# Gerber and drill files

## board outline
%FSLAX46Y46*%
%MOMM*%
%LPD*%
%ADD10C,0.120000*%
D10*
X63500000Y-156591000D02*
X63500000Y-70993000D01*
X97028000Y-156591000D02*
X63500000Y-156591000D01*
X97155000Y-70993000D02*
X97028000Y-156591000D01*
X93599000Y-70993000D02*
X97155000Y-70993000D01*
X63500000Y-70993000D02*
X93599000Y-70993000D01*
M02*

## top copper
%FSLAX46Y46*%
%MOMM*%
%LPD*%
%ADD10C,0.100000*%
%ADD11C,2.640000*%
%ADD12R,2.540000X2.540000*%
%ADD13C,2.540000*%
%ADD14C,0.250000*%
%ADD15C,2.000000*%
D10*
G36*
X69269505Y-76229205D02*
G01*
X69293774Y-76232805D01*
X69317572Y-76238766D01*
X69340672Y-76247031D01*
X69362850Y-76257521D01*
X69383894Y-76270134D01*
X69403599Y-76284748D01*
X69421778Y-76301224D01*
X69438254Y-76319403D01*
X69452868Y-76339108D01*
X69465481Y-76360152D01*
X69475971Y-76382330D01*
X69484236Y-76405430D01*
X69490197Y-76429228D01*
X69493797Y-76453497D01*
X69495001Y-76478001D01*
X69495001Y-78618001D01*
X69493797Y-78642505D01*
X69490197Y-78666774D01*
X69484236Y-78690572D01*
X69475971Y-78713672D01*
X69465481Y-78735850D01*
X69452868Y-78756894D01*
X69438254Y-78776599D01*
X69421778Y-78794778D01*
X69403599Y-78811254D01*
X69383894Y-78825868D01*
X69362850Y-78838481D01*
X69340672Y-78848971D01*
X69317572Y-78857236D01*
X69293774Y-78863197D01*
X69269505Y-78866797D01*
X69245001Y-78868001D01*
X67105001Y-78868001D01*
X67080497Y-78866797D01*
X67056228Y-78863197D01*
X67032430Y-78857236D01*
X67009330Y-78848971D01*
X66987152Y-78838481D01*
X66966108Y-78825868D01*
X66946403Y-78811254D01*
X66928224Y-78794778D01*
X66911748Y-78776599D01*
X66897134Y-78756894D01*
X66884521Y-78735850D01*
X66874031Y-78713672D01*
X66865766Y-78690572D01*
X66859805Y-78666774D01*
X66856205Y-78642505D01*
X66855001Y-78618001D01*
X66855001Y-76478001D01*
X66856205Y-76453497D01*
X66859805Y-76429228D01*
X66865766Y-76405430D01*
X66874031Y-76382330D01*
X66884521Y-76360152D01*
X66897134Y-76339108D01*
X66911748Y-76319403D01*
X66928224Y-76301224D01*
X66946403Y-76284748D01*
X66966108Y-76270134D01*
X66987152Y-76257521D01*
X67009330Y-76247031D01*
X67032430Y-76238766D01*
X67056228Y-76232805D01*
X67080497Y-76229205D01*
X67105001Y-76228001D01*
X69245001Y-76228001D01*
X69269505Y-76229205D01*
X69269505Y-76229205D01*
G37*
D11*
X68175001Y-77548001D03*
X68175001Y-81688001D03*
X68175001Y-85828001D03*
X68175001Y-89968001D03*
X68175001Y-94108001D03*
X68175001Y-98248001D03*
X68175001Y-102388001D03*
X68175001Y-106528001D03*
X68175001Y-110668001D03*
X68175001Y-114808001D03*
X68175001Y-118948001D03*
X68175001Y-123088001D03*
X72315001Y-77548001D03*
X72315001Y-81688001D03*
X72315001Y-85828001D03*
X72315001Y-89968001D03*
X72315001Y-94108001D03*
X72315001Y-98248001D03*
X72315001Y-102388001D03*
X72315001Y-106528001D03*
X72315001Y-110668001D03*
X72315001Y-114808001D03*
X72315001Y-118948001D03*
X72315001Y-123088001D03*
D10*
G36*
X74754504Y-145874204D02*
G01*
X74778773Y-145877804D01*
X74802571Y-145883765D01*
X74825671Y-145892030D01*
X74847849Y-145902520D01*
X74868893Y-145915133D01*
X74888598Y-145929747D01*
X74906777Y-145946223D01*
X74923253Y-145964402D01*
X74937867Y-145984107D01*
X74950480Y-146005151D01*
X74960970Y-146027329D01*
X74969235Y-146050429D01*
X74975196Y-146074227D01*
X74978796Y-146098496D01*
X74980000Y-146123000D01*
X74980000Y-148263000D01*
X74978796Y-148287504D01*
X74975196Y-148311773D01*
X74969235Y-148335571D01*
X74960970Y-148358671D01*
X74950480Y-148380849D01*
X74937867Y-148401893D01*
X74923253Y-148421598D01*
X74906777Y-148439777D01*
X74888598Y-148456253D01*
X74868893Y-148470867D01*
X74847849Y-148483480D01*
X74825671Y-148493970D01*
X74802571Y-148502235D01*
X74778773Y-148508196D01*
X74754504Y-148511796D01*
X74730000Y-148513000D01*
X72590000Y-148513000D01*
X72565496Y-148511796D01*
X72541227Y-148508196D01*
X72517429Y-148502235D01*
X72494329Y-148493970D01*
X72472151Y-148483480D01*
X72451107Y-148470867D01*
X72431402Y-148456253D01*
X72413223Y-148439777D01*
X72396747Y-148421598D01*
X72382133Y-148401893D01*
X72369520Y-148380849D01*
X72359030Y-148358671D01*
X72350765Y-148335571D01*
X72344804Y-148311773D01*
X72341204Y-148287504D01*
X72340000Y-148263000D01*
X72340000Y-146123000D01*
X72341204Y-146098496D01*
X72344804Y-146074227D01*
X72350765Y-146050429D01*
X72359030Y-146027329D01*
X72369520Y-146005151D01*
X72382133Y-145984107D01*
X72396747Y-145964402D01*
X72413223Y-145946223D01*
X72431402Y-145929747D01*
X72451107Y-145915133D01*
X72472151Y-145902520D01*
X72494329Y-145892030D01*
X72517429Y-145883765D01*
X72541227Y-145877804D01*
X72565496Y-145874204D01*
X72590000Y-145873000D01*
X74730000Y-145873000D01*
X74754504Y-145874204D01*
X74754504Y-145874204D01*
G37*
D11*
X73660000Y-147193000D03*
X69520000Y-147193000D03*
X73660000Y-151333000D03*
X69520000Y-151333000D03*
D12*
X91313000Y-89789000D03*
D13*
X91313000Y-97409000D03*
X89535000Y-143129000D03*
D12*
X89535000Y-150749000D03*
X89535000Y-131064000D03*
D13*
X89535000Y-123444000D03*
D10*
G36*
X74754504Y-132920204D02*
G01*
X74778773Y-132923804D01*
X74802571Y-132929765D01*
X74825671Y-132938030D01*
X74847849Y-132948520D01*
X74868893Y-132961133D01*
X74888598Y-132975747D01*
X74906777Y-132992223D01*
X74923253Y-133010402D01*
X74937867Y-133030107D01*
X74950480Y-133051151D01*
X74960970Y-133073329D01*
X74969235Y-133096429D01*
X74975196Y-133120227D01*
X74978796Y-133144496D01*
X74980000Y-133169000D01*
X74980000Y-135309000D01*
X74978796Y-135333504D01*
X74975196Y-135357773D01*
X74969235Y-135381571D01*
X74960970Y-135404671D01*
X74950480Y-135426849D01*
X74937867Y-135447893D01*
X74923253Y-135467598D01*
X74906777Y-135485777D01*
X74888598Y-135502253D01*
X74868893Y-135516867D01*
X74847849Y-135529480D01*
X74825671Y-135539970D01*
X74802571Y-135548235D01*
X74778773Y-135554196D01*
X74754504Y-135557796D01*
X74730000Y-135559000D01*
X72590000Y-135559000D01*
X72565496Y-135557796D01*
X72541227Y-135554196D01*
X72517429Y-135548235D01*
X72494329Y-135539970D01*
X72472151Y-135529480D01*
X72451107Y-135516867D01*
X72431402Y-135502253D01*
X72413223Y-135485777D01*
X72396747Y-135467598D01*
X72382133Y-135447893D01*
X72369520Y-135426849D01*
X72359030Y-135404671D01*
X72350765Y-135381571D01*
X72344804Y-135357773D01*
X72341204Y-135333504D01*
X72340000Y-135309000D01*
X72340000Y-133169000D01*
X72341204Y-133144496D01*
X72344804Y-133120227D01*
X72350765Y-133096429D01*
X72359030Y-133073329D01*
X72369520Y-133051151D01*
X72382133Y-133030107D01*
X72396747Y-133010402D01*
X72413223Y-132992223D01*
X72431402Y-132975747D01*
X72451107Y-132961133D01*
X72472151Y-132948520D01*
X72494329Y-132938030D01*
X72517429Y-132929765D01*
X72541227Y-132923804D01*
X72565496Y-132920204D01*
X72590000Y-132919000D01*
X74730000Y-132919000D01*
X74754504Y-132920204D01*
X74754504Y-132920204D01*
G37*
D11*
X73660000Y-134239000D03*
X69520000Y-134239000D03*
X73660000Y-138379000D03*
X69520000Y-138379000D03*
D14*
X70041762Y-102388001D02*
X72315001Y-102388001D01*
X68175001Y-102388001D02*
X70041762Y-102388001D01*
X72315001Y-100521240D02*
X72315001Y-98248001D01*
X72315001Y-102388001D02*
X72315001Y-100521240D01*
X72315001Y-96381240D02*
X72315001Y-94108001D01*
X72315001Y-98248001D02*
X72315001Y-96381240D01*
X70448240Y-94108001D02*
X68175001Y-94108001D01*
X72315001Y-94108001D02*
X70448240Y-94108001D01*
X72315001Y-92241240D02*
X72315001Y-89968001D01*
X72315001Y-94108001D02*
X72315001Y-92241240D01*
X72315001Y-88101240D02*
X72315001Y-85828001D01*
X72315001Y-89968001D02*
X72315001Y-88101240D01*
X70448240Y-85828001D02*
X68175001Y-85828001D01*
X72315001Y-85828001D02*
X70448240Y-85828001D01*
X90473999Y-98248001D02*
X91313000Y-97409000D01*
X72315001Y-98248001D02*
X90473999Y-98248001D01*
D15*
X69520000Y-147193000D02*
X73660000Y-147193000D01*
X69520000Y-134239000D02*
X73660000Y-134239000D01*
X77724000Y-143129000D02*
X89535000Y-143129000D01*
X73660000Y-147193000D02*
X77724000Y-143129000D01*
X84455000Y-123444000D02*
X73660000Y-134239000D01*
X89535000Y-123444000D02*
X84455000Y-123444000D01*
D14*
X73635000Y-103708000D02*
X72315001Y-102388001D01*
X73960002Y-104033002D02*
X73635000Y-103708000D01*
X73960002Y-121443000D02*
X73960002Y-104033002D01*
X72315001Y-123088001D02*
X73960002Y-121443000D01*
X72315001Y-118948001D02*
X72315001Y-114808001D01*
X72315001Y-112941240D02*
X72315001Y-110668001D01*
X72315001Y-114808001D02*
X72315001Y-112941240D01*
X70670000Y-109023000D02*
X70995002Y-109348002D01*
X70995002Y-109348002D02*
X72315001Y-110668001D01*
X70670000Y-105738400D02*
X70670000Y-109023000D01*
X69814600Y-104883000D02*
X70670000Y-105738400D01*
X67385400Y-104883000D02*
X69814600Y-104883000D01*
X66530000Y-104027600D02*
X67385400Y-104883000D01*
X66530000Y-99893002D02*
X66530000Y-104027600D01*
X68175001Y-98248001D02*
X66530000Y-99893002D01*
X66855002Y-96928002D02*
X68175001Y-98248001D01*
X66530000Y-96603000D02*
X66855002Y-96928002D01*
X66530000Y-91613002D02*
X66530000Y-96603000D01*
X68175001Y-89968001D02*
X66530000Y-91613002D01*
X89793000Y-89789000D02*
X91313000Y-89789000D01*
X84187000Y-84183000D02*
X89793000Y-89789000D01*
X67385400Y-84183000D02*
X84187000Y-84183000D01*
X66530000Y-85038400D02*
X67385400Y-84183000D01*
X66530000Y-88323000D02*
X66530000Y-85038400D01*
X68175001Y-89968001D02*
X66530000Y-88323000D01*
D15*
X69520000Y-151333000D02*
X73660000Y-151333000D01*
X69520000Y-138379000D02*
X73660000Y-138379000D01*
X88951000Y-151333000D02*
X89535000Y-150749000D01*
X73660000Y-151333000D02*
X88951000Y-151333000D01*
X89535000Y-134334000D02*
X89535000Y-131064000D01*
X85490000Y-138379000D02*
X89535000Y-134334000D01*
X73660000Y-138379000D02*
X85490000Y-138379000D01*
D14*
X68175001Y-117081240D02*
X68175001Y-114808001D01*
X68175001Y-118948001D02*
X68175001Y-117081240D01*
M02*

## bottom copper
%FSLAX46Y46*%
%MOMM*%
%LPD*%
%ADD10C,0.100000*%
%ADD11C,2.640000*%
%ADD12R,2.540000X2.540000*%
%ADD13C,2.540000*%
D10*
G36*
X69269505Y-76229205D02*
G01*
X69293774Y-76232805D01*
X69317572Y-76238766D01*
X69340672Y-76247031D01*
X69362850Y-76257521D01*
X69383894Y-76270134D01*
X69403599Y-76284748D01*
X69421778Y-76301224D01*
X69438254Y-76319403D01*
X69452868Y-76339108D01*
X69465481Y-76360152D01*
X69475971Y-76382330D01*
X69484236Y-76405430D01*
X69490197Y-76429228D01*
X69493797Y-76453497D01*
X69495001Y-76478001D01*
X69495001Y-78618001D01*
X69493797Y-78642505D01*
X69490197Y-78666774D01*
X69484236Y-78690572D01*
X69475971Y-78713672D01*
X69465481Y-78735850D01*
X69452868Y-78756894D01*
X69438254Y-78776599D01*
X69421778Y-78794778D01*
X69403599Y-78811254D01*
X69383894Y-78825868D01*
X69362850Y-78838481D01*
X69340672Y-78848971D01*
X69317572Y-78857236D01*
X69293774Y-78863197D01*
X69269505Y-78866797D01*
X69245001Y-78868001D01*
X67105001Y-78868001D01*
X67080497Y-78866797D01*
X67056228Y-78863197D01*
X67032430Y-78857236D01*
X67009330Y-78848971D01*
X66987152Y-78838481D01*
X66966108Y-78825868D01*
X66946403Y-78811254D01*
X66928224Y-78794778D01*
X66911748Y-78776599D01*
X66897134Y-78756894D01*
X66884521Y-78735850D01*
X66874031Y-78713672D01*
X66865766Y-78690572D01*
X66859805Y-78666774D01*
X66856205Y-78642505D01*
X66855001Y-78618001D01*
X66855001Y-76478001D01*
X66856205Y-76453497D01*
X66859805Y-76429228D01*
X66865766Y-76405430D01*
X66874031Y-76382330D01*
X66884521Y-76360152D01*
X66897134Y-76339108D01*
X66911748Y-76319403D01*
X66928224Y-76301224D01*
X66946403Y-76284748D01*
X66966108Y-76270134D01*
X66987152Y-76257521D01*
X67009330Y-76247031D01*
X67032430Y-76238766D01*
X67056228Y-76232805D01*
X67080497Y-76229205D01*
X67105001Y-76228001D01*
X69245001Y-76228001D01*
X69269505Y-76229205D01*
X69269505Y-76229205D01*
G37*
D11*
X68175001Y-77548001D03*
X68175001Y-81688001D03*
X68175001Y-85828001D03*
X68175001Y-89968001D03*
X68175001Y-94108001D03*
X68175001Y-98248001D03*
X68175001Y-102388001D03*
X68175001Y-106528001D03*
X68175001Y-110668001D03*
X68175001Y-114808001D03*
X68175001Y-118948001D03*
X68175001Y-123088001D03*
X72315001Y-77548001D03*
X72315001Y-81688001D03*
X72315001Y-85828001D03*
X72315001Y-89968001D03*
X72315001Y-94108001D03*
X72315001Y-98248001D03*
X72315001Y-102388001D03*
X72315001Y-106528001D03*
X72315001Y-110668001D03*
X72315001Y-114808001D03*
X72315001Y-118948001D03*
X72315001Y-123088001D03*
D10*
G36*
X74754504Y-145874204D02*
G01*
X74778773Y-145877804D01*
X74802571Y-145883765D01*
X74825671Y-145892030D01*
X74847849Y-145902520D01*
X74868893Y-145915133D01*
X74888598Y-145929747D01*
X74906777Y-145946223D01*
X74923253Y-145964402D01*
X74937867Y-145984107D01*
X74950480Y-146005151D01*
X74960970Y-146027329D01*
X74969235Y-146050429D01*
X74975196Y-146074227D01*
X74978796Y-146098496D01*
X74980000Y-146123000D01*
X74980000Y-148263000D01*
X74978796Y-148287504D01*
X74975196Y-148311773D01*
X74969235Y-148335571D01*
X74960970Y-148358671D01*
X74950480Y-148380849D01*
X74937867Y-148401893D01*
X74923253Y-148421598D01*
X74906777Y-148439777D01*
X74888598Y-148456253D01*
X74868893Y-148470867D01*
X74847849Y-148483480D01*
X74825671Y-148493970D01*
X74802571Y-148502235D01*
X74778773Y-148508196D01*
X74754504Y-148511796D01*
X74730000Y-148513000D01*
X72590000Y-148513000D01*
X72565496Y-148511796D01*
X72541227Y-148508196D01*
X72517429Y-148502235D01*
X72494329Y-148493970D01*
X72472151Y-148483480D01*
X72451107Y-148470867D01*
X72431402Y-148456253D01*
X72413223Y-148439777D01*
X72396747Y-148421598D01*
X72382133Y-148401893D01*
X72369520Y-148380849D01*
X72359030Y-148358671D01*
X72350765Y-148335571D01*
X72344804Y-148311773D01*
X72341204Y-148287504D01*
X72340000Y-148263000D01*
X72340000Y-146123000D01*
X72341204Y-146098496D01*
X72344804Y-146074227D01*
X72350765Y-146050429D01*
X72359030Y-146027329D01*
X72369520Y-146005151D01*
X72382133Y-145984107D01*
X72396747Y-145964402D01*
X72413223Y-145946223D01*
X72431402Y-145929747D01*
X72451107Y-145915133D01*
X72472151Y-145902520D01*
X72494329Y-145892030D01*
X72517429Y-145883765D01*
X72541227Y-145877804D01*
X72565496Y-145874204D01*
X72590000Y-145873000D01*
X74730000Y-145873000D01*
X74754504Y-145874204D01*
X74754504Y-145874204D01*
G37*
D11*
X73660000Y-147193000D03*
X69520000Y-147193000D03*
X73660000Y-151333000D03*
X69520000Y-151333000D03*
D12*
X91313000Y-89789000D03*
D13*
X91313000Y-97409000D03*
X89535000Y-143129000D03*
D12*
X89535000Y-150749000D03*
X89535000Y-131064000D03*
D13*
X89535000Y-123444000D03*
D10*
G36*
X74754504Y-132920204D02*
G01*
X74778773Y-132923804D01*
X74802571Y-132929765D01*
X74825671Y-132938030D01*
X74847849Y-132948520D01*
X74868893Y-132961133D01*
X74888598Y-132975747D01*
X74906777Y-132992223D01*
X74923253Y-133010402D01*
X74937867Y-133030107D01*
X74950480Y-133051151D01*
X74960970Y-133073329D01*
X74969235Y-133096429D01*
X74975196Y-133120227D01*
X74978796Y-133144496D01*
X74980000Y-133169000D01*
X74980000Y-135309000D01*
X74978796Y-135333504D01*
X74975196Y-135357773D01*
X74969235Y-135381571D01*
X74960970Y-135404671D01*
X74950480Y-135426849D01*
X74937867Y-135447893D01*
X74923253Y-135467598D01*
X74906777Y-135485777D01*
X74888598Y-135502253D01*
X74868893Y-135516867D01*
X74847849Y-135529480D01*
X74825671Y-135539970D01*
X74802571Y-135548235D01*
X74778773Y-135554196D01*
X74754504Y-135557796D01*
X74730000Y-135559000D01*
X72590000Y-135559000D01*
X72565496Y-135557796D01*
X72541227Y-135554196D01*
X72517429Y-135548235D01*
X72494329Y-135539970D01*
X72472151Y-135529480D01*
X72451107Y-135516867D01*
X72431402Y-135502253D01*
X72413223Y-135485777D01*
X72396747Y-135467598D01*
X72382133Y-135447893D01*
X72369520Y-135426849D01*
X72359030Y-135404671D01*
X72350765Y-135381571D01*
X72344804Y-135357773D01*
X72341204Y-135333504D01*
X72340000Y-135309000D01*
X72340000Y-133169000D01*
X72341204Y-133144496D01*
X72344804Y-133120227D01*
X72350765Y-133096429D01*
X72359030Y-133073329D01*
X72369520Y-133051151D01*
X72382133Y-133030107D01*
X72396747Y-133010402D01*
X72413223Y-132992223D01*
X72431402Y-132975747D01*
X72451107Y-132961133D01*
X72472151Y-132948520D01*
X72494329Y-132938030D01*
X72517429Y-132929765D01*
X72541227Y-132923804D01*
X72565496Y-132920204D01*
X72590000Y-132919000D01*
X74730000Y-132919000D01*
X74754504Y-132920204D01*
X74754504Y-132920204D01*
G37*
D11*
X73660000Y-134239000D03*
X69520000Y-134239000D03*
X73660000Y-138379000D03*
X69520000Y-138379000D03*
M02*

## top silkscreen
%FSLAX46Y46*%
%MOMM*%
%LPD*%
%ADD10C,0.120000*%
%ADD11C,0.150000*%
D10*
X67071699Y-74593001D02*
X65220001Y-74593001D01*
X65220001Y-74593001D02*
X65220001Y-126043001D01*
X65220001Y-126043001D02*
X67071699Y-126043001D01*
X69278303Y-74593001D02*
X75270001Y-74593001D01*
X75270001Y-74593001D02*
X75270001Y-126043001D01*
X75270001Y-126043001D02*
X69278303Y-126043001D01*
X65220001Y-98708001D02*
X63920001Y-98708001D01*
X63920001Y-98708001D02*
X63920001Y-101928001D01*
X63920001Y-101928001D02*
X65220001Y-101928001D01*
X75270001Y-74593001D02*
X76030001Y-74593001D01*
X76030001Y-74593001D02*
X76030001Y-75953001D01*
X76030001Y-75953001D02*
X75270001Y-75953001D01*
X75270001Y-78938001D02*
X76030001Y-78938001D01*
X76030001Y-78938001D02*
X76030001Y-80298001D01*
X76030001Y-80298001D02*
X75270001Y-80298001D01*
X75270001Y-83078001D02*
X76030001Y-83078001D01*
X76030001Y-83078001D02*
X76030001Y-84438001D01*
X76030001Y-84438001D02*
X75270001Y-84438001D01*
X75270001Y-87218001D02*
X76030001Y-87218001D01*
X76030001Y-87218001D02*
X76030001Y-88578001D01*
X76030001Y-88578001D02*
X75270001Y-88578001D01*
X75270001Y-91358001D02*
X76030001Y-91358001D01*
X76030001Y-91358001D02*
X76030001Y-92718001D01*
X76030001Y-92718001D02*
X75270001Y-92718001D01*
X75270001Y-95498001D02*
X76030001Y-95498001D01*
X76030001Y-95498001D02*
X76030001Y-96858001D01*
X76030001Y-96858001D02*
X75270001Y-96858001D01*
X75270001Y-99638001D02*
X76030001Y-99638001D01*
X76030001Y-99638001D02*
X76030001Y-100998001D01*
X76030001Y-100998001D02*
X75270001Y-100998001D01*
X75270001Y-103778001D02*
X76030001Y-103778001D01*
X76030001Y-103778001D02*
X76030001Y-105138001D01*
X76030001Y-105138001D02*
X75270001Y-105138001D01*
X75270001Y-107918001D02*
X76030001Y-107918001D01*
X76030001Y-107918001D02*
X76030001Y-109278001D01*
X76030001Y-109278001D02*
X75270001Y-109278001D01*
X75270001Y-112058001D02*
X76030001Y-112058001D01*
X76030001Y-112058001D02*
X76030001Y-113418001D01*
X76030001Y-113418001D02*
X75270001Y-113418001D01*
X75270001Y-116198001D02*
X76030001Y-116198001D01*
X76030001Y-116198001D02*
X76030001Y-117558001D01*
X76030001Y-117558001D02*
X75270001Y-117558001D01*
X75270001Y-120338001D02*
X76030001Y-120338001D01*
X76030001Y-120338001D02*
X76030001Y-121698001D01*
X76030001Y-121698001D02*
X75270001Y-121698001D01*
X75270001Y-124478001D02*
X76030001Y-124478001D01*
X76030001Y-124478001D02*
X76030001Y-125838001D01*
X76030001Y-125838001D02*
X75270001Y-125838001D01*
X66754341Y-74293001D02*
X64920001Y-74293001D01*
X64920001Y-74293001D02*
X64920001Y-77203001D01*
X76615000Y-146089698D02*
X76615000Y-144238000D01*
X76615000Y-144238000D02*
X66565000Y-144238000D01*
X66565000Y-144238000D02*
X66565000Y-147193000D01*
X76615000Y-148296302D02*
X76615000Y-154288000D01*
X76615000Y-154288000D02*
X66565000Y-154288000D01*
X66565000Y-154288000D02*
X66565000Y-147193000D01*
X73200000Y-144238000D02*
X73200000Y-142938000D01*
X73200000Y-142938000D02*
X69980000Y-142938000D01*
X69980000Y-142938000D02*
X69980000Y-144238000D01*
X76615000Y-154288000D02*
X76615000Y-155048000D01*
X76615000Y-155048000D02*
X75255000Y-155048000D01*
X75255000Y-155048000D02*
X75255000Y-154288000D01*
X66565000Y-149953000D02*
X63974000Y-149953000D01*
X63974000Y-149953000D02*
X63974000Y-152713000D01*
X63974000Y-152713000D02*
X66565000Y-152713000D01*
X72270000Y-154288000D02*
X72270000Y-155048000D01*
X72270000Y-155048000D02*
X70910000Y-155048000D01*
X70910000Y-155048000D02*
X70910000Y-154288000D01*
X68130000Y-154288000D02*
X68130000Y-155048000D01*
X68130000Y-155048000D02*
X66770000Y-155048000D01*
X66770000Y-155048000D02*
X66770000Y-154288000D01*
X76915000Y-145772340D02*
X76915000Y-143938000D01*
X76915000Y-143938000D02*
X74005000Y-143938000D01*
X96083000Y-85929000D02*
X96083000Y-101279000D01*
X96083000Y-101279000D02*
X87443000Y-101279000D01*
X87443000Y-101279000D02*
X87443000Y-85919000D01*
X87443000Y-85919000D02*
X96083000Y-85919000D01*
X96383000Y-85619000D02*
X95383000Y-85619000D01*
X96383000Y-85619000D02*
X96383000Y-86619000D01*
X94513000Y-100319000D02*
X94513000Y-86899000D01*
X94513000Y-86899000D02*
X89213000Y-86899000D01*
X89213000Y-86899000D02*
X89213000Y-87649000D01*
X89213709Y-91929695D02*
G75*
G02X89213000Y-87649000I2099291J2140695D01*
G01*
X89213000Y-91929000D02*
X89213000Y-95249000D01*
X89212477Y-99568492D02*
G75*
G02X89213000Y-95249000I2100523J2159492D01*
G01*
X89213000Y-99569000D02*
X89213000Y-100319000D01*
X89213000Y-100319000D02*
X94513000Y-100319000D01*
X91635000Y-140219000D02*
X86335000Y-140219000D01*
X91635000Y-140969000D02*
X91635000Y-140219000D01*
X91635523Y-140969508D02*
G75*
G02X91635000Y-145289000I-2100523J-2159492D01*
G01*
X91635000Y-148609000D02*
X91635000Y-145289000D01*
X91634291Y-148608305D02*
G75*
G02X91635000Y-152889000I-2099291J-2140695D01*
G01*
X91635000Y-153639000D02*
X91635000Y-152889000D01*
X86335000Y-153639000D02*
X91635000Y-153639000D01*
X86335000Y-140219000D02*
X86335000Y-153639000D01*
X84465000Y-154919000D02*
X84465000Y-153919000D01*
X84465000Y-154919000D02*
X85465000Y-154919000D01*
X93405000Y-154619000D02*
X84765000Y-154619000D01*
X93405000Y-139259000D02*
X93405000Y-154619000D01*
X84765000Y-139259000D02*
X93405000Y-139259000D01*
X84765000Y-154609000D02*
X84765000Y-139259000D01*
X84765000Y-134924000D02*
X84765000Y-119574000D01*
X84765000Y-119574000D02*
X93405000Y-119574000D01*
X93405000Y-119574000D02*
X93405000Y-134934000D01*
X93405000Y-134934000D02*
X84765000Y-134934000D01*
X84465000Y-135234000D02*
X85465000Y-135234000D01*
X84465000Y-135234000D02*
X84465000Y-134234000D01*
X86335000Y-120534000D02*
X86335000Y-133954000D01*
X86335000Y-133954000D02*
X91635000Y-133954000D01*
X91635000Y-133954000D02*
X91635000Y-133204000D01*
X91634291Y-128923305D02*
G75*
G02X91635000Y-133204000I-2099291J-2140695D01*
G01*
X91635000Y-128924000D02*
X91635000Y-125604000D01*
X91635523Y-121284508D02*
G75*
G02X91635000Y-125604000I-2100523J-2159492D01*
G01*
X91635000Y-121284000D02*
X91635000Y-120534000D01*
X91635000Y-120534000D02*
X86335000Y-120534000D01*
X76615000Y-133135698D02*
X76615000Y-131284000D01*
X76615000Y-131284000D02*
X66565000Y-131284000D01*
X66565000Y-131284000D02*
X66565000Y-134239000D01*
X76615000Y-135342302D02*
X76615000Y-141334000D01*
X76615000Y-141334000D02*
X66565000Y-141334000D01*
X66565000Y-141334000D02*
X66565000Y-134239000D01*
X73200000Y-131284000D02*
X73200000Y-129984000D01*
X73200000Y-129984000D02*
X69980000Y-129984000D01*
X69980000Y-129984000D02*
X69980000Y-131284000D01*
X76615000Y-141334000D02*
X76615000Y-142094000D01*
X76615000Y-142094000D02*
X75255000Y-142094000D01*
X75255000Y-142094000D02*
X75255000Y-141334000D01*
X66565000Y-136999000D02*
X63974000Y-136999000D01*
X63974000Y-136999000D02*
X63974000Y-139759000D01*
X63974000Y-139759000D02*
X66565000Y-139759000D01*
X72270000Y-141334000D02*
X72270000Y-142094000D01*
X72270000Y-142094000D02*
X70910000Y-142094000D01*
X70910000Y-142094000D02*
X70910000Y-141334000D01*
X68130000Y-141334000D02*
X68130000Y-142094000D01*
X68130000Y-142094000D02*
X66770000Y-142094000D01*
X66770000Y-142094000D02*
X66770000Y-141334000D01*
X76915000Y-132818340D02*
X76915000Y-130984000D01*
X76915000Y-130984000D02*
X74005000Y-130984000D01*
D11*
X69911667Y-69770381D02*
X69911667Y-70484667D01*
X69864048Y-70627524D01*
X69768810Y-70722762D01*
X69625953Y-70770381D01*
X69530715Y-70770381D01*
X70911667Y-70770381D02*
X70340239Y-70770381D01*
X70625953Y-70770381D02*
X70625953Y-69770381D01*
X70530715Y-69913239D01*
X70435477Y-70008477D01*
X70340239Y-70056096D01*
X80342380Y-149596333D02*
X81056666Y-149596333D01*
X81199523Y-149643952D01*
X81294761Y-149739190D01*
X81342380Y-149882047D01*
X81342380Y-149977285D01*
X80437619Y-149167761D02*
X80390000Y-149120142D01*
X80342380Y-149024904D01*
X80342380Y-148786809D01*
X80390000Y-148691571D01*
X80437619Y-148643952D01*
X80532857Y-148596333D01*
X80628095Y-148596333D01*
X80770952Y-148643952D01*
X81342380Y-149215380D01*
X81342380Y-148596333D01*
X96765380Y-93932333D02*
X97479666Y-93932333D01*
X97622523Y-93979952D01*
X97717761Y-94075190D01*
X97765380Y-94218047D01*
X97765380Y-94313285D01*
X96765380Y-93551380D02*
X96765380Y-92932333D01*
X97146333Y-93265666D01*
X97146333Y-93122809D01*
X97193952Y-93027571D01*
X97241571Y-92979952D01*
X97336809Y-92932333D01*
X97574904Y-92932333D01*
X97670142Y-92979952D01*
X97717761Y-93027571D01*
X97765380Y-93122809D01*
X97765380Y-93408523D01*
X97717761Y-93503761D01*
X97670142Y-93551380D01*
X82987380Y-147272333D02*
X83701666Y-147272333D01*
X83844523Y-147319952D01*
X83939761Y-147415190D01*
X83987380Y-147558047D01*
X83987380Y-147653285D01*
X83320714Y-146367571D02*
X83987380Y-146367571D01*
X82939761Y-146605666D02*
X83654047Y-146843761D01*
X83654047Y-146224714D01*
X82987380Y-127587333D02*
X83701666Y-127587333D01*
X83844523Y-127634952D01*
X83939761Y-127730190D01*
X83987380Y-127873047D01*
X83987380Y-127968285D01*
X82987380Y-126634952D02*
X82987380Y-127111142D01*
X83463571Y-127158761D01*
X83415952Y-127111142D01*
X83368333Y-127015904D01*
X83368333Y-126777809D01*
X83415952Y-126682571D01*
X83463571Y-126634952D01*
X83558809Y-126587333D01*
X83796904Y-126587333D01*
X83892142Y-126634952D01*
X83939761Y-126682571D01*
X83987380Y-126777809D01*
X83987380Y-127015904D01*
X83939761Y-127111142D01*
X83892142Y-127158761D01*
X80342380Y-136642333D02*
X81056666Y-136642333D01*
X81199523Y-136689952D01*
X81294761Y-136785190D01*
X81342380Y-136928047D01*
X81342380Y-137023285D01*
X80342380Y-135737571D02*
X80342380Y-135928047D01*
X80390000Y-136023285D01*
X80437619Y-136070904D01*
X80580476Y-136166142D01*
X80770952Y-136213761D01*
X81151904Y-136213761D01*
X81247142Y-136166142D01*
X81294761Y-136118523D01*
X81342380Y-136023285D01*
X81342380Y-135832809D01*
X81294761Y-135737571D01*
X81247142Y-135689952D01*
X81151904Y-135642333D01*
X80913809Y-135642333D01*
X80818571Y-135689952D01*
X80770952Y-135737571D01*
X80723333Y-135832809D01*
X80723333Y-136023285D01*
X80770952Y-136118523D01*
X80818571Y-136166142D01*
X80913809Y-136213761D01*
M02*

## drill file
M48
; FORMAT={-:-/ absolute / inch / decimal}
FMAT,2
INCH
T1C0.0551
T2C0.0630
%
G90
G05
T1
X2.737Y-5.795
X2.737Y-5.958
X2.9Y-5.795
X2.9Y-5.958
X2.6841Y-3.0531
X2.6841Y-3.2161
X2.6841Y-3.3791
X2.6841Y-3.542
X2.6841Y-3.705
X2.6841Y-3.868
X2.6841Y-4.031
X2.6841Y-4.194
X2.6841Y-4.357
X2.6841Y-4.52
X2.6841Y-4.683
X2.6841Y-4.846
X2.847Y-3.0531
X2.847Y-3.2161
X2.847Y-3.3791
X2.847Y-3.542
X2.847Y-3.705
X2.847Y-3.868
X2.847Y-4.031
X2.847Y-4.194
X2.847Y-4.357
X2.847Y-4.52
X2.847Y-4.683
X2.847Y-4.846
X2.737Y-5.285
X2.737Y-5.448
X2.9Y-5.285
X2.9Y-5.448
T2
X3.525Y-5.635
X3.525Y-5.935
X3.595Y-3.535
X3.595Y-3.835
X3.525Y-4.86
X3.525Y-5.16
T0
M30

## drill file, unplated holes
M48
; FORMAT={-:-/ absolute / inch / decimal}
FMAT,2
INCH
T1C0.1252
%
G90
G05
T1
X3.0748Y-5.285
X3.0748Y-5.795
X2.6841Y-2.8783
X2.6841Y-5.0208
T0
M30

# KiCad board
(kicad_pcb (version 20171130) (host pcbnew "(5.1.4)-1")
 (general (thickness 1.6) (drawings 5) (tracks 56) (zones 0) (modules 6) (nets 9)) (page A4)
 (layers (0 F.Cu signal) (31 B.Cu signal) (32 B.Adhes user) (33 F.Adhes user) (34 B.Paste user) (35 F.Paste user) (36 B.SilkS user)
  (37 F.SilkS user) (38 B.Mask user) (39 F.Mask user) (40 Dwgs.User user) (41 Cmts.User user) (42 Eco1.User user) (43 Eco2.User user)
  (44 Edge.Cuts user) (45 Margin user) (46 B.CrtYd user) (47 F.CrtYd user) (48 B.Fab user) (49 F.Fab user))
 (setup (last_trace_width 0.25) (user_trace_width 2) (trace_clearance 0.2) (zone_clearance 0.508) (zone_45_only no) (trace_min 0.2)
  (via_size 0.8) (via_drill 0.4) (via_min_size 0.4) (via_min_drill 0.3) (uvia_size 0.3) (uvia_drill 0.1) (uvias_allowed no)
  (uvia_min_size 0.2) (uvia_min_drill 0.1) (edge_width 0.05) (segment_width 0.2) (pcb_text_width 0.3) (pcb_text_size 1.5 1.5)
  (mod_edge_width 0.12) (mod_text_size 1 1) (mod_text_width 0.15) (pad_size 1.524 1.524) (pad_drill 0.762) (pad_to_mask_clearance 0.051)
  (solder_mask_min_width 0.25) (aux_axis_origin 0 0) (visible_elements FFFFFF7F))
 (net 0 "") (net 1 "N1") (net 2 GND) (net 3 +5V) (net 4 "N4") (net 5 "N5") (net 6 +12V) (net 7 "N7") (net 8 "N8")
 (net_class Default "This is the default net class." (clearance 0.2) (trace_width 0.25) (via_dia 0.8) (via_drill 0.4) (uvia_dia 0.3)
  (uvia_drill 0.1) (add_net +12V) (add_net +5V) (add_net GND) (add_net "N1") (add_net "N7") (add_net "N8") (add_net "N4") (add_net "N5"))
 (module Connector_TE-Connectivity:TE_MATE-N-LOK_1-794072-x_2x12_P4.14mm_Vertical (layer F.Cu) (at 68.175001 77.548001)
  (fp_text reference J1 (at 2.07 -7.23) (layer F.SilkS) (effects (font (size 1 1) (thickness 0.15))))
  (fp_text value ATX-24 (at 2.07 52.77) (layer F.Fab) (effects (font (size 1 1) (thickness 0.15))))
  (fp_line (start -1.103302 -2.955) (end -2.955 -2.955) (layer F.SilkS) (width 0.12))
  (fp_line (start -2.955 -2.955) (end -2.955 48.495) (layer F.SilkS) (width 0.12))
  (fp_line (start -2.955 48.495) (end -1.103302 48.495) (layer F.SilkS) (width 0.12))
  (fp_line (start 1.103302 -2.955) (end 7.095 -2.955) (layer F.SilkS) (width 0.12))
  (fp_line (start 7.095 -2.955) (end 7.095 48.495) (layer F.SilkS) (width 0.12))
  (fp_line (start 7.095 48.495) (end 1.103302 48.495) (layer F.SilkS) (width 0.12))
  (fp_line (start -2.955 21.16) (end -4.255 21.16) (layer F.SilkS) (width 0.12))
  (fp_line (start -4.255 21.16) (end -4.255 24.38) (layer F.SilkS) (width 0.12))
  (fp_line (start -4.255 24.38) (end -2.955 24.38) (layer F.SilkS) (width 0.12))
  (fp_line (start 7.095 -2.955) (end 7.855 -2.955) (layer F.SilkS) (width 0.12))
  (fp_line (start 7.855 -2.955) (end 7.855 -1.595) (layer F.SilkS) (width 0.12))
  (fp_line (start 7.855 -1.595) (end 7.095 -1.595) (layer F.SilkS) (width 0.12))
  (fp_line (start 7.095 1.39) (end 7.855 1.39) (layer F.SilkS) (width 0.12))
  (fp_line (start 7.855 1.39) (end 7.855 2.75) (layer F.SilkS) (width 0.12))
  (fp_line (start 7.855 2.75) (end 7.095 2.75) (layer F.SilkS) (width 0.12))
  (fp_line (start 7.095 5.53) (end 7.855 5.53) (layer F.SilkS) (width 0.12))
  (fp_line (start 7.855 5.53) (end 7.855 6.89) (layer F.SilkS) (width 0.12))
  (fp_line (start 7.855 6.89) (end 7.095 6.89) (layer F.SilkS) (width 0.12))
  (fp_line (start 7.095 9.67) (end 7.855 9.67) (layer F.SilkS) (width 0.12))
  (fp_line (start 7.855 9.67) (end 7.855 11.03) (layer F.SilkS) (width 0.12))
  (fp_line (start 7.855 11.03) (end 7.095 11.03) (layer F.SilkS) (width 0.12))
  (fp_line (start 7.095 13.81) (end 7.855 13.81) (layer F.SilkS) (width 0.12))
  (fp_line (start 7.855 13.81) (end 7.855 15.17) (layer F.SilkS) (width 0.12))
  (fp_line (start 7.855 15.17) (end 7.095 15.17) (layer F.SilkS) (width 0.12))
  (fp_line (start 7.095 17.95) (end 7.855 17.95) (layer F.SilkS) (width 0.12))
  (fp_line (start 7.855 17.95) (end 7.855 19.31) (layer F.SilkS) (width 0.12))
  (fp_line (start 7.855 19.31) (end 7.095 19.31) (layer F.SilkS) (width 0.12))
  (fp_line (start 7.095 22.09) (end 7.855 22.09) (layer F.SilkS) (width 0.12))
  (fp_line (start 7.855 22.09) (end 7.855 23.45) (layer F.SilkS) (width 0.12))
  (fp_line (start 7.855 23.45) (end 7.095 23.45) (layer F.SilkS) (width 0.12))
  (fp_line (start 7.095 26.23) (end 7.855 26.23) (layer F.SilkS) (width 0.12))
  (fp_line (start 7.855 26.23) (end 7.855 27.59) (layer F.SilkS) (width 0.12))
  (fp_line (start 7.855 27.59) (end 7.095 27.59) (layer F.SilkS) (width 0.12))
  (fp_line (start 7.095 30.37) (end 7.855 30.37) (layer F.SilkS) (width 0.12))
  (fp_line (start 7.855 30.37) (end 7.855 31.73) (layer F.SilkS) (width 0.12))
  (fp_line (start 7.855 31.73) (end 7.095 31.73) (layer F.SilkS) (width 0.12))
  (fp_line (start 7.095 34.51) (end 7.855 34.51) (layer F.SilkS) (width 0.12))
  (fp_line (start 7.855 34.51) (end 7.855 35.87) (layer F.SilkS) (width 0.12))
  (fp_line (start 7.855 35.87) (end 7.095 35.87) (layer F.SilkS) (width 0.12))
  (fp_line (start 7.095 38.65) (end 7.855 38.65) (layer F.SilkS) (width 0.12))
  (fp_line (start 7.855 38.65) (end 7.855 40.01) (layer F.SilkS) (width 0.12))
  (fp_line (start 7.855 40.01) (end 7.095 40.01) (layer F.SilkS) (width 0.12))
  (fp_line (start 7.095 42.79) (end 7.855 42.79) (layer F.SilkS) (width 0.12))
  (fp_line (start 7.855 42.79) (end 7.855 44.15) (layer F.SilkS) (width 0.12))
  (fp_line (start 7.855 44.15) (end 7.095 44.15) (layer F.SilkS) (width 0.12))
  (fp_line (start 7.095 46.93) (end 7.855 46.93) (layer F.SilkS) (width 0.12))
  (fp_line (start 7.855 46.93) (end 7.855 48.29) (layer F.SilkS) (width 0.12))
  (fp_line (start 7.855 48.29) (end 7.095 48.29) (layer F.SilkS) (width 0.12))
  (fp_line (start -1.42066 -3.255) (end -3.255 -3.255) (layer F.SilkS) (width 0.12))
  (fp_line (start -3.255 -3.255) (end -3.255 -0.345) (layer F.SilkS) (width 0.12))
  (pad 1 thru_hole roundrect (at 0 0) (size 2.64 2.64) (drill 1.4) (layers *.Cu *.Mask) (roundrect_rratio 0.094697) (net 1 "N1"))
  (pad 2 thru_hole circle (at 0 4.14) (size 2.64 2.64) (drill 1.4) (layers *.Cu *.Mask) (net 1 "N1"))
  (pad 3 thru_hole circle (at 0 8.28) (size 2.64 2.64) (drill 1.4) (layers *.Cu *.Mask) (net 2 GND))
  (pad 4 thru_hole circle (at 0 12.42) (size 2.64 2.64) (drill 1.4) (layers *.Cu *.Mask) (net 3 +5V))
  (pad 5 thru_hole circle (at 0 16.56) (size 2.64 2.64) (drill 1.4) (layers *.Cu *.Mask) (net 2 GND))
  (pad 6 thru_hole circle (at 0 20.7) (size 2.64 2.64) (drill 1.4) (layers *.Cu *.Mask) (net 3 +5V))
  (pad 7 thru_hole circle (at 0 24.84) (size 2.64 2.64) (drill 1.4) (layers *.Cu *.Mask) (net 2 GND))
  (pad 8 thru_hole circle (at 0 28.98) (size 2.64 2.64) (drill 1.4) (layers *.Cu *.Mask) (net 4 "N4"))
  (pad 9 thru_hole circle (at 0 33.12) (size 2.64 2.64) (drill 1.4) (layers *.Cu *.Mask) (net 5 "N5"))
  (pad 10 thru_hole circle (at 0 37.26) (size 2.64 2.64) (drill 1.4) (layers *.Cu *.Mask) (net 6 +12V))
  (pad 11 thru_hole circle (at 0 41.4) (size 2.64 2.64) (drill 1.4) (layers *.Cu *.Mask) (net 6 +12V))
  (pad 12 thru_hole circle (at 0 45.54) (size 2.64 2.64) (drill 1.4) (layers *.Cu *.Mask) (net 1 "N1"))
  (pad 13 thru_hole circle (at 4.14 0) (size 2.64 2.64) (drill 1.4) (layers *.Cu *.Mask) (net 1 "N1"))
  (pad 14 thru_hole circle (at 4.14 4.14) (size 2.64 2.64) (drill 1.4) (layers *.Cu *.Mask) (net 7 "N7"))
  (pad 15 thru_hole circle (at 4.14 8.28) (size 2.64 2.64) (drill 1.4) (layers *.Cu *.Mask) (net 2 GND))
  (pad 16 thru_hole circle (at 4.14 12.42) (size 2.64 2.64) (drill 1.4) (layers *.Cu *.Mask) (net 2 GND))
  (pad 17 thru_hole circle (at 4.14 16.56) (size 2.64 2.64) (drill 1.4) (layers *.Cu *.Mask) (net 2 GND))
  (pad 18 thru_hole circle (at 4.14 20.7) (size 2.64 2.64) (drill 1.4) (layers *.Cu *.Mask) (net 2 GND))
  (pad 19 thru_hole circle (at 4.14 24.84) (size 2.64 2.64) (drill 1.4) (layers *.Cu *.Mask) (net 2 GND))
  (pad 20 thru_hole circle (at 4.14 28.98) (size 2.64 2.64) (drill 1.4) (layers *.Cu *.Mask) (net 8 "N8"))
  (pad 21 thru_hole circle (at 4.14 33.12) (size 2.64 2.64) (drill 1.4) (layers *.Cu *.Mask) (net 3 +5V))
  (pad 22 thru_hole circle (at 4.14 37.26) (size 2.64 2.64) (drill 1.4) (layers *.Cu *.Mask) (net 3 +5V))
  (pad 23 thru_hole circle (at 4.14 41.4) (size 2.64 2.64) (drill 1.4) (layers *.Cu *.Mask) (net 3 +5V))
  (pad 24 thru_hole circle (at 4.14 45.54) (size 2.64 2.64) (drill 1.4) (layers *.Cu *.Mask) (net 2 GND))
  (pad "" np_thru_hole circle (at 0 -4.44) (size 3.18 3.18) (drill 3.18) (layers *.Cu *.Mask))
  (pad "" np_thru_hole circle (at 0 49.98) (size 3.18 3.18) (drill 3.18) (layers *.Cu *.Mask)))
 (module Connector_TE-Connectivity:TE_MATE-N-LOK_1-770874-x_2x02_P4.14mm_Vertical (layer F.Cu) (at 73.66 147.193 270)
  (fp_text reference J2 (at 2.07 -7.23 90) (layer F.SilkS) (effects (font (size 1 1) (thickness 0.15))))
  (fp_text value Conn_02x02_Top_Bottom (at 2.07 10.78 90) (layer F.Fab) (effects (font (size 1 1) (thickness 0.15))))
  (fp_line (start -1.103302 -2.955) (end -2.955 -2.955) (layer F.SilkS) (width 0.12))
  (fp_line (start -2.955 -2.955) (end -2.955 7.095) (layer F.SilkS) (width 0.12))
  (fp_line (start -2.955 7.095) (end 0 7.095) (layer F.SilkS) (width 0.12))
  (fp_line (start 1.103302 -2.955) (end 7.095 -2.955) (layer F.SilkS) (width 0.12))
  (fp_line (start 7.095 -2.955) (end 7.095 7.095) (layer F.SilkS) (width 0.12))
  (fp_line (start 7.095 7.095) (end 0 7.095) (layer F.SilkS) (width 0.12))
  (fp_line (start -2.955 0.46) (end -4.255 0.46) (layer F.SilkS) (width 0.12))
  (fp_line (start -4.255 0.46) (end -4.255 3.68) (layer F.SilkS) (width 0.12))
  (fp_line (start -4.255 3.68) (end -2.955 3.68) (layer F.SilkS) (width 0.12))
  (fp_line (start 7.095 -2.955) (end 7.855 -2.955) (layer F.SilkS) (width 0.12))
  (fp_line (start 7.855 -2.955) (end 7.855 -1.595) (layer F.SilkS) (width 0.12))
  (fp_line (start 7.855 -1.595) (end 7.095 -1.595) (layer F.SilkS) (width 0.12))
  (fp_line (start 2.76 7.095) (end 2.76 9.686) (layer F.SilkS) (width 0.12))
  (fp_line (start 2.76 9.686) (end 5.52 9.686) (layer F.SilkS) (width 0.12))
  (fp_line (start 5.52 9.686) (end 5.52 7.095) (layer F.SilkS) (width 0.12))
  (fp_line (start 7.095 1.39) (end 7.855 1.39) (layer F.SilkS) (width 0.12))
  (fp_line (start 7.855 1.39) (end 7.855 2.75) (layer F.SilkS) (width 0.12))
  (fp_line (start 7.855 2.75) (end 7.095 2.75) (layer F.SilkS) (width 0.12))
  (fp_line (start 7.095 5.53) (end 7.855 5.53) (layer F.SilkS) (width 0.12))
  (fp_line (start 7.855 5.53) (end 7.855 6.89) (layer F.SilkS) (width 0.12))
  (fp_line (start 7.855 6.89) (end 7.095 6.89) (layer F.SilkS) (width 0.12))
  (fp_line (start -1.42066 -3.255) (end -3.255 -3.255) (layer F.SilkS) (width 0.12))
  (fp_line (start -3.255 -3.255) (end -3.255 -0.345) (layer F.SilkS) (width 0.12))
  (pad 1 thru_hole roundrect (at 0 0 270) (size 2.64 2.64) (drill 1.4) (layers *.Cu *.Mask) (roundrect_rratio 0.094697) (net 2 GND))
  (pad 2 thru_hole circle (at 0 4.14 270) (size 2.64 2.64) (drill 1.4) (layers *.Cu *.Mask) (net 2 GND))
  (pad 3 thru_hole circle (at 4.14 0 270) (size 2.64 2.64) (drill 1.4) (layers *.Cu *.Mask) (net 6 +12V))
  (pad 4 thru_hole circle (at 4.14 4.14 270) (size 2.64 2.64) (drill 1.4) (layers *.Cu *.Mask) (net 6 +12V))
  (pad "" np_thru_hole circle (at 0 -4.44 270) (size 3.18 3.18) (drill 3.18) (layers *.Cu *.Mask)))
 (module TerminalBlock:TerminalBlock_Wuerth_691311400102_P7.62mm (layer F.Cu) (at 91.313 89.789 270)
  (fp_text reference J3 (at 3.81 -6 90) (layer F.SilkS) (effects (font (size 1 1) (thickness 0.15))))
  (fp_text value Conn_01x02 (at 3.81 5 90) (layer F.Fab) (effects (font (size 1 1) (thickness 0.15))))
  (fp_line (start -3.86 -4.77) (end 11.49 -4.77) (layer F.SilkS) (width 0.12))
  (fp_line (start 11.49 -4.77) (end 11.49 3.87) (layer F.SilkS) (width 0.12))
  (fp_line (start 11.49 3.87) (end -3.87 3.87) (layer F.SilkS) (width 0.12))
  (fp_line (start -3.87 3.87) (end -3.87 -4.77) (layer F.SilkS) (width 0.12))
  (fp_line (start -4.17 -5.07) (end -4.17 -4.07) (layer F.SilkS) (width 0.12))
  (fp_line (start -4.17 -5.07) (end -3.17 -5.07) (layer F.SilkS) (width 0.12))
  (fp_line (start 10.53 -3.2) (end -2.89 -3.2) (layer F.SilkS) (width 0.12))
  (fp_line (start -2.89 -3.2) (end -2.89 2.1) (layer F.SilkS) (width 0.12))
  (fp_line (start -2.89 2.1) (end -2.14 2.1) (layer F.SilkS) (width 0.12))
  (fp_arc (start 0 0) (end -2.14 2.1) (angle -91.1) (layer F.SilkS) (width 0.12))
  (fp_line (start 2.14 2.1) (end 5.46 2.1) (layer F.SilkS) (width 0.12))
  (fp_arc (start 7.62 0) (end 5.46 2.1) (angle -91.6) (layer F.SilkS) (width 0.12))
  (fp_line (start 9.78 2.1) (end 10.53 2.1) (layer F.SilkS) (width 0.12))
  (fp_line (start 10.53 2.1) (end 10.53 -3.2) (layer F.SilkS) (width 0.12))
  (pad 1 thru_hole rect (at 0 0 270) (size 2.54 2.54) (drill 1.6) (layers *.Cu *.Mask) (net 3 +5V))
  (pad 2 thru_hole circle (at 7.62 0 270) (size 2.54 2.54) (drill 1.6) (layers *.Cu *.Mask) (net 2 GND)))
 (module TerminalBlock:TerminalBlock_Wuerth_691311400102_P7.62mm (layer F.Cu) (at 89.535 150.749 90)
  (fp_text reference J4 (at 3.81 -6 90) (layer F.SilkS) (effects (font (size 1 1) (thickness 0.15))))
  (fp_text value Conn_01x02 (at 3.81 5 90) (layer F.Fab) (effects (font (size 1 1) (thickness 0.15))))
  (fp_line (start 10.53 2.1) (end 10.53 -3.2) (layer F.SilkS) (width 0.12))
  (fp_line (start 9.78 2.1) (end 10.53 2.1) (layer F.SilkS) (width 0.12))
  (fp_arc (start 7.62 0) (end 5.46 2.1) (angle -91.6) (layer F.SilkS) (width 0.12))
  (fp_line (start 2.14 2.1) (end 5.46 2.1) (layer F.SilkS) (width 0.12))
  (fp_arc (start 0 0) (end -2.14 2.1) (angle -91.1) (layer F.SilkS) (width 0.12))
  (fp_line (start -2.89 2.1) (end -2.14 2.1) (layer F.SilkS) (width 0.12))
  (fp_line (start -2.89 -3.2) (end -2.89 2.1) (layer F.SilkS) (width 0.12))
  (fp_line (start 10.53 -3.2) (end -2.89 -3.2) (layer F.SilkS) (width 0.12))
  (fp_line (start -4.17 -5.07) (end -3.17 -5.07) (layer F.SilkS) (width 0.12))
  (fp_line (start -4.17 -5.07) (end -4.17 -4.07) (layer F.SilkS) (width 0.12))
  (fp_line (start -3.87 3.87) (end -3.87 -4.77) (layer F.SilkS) (width 0.12))
  (fp_line (start 11.49 3.87) (end -3.87 3.87) (layer F.SilkS) (width 0.12))
  (fp_line (start 11.49 -4.77) (end 11.49 3.87) (layer F.SilkS) (width 0.12))
  (fp_line (start -3.86 -4.77) (end 11.49 -4.77) (layer F.SilkS) (width 0.12))
  (pad 2 thru_hole circle (at 7.62 0 90) (size 2.54 2.54) (drill 1.6) (layers *.Cu *.Mask) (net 2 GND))
  (pad 1 thru_hole rect (at 0 0 90) (size 2.54 2.54) (drill 1.6) (layers *.Cu *.Mask) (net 6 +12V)))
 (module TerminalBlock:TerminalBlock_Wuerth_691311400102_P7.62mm (layer F.Cu) (at 89.535 131.064 90)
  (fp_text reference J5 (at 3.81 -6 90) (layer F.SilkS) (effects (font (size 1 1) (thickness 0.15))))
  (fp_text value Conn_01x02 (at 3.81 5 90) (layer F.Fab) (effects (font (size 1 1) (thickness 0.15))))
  (fp_line (start -3.86 -4.77) (end 11.49 -4.77) (layer F.SilkS) (width 0.12))
  (fp_line (start 11.49 -4.77) (end 11.49 3.87) (layer F.SilkS) (width 0.12))
  (fp_line (start 11.49 3.87) (end -3.87 3.87) (layer F.SilkS) (width 0.12))
  (fp_line (start -3.87 3.87) (end -3.87 -4.77) (layer F.SilkS) (width 0.12))
  (fp_line (start -4.17 -5.07) (end -4.17 -4.07) (layer F.SilkS) (width 0.12))
  (fp_line (start -4.17 -5.07) (end -3.17 -5.07) (layer F.SilkS) (width 0.12))
  (fp_line (start 10.53 -3.2) (end -2.89 -3.2) (layer F.SilkS) (width 0.12))
  (fp_line (start -2.89 -3.2) (end -2.89 2.1) (layer F.SilkS) (width 0.12))
  (fp_line (start -2.89 2.1) (end -2.14 2.1) (layer F.SilkS) (width 0.12))
  (fp_arc (start 0 0) (end -2.14 2.1) (angle -91.1) (layer F.SilkS) (width 0.12))
  (fp_line (start 2.14 2.1) (end 5.46 2.1) (layer F.SilkS) (width 0.12))
  (fp_arc (start 7.62 0) (end 5.46 2.1) (angle -91.6) (layer F.SilkS) (width 0.12))
  (fp_line (start 9.78 2.1) (end 10.53 2.1) (layer F.SilkS) (width 0.12))
  (fp_line (start 10.53 2.1) (end 10.53 -3.2) (layer F.SilkS) (width 0.12))
  (pad 1 thru_hole rect (at 0 0 90) (size 2.54 2.54) (drill 1.6) (layers *.Cu *.Mask) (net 6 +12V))
  (pad 2 thru_hole circle (at 7.62 0 90) (size 2.54 2.54) (drill 1.6) (layers *.Cu *.Mask) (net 2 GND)))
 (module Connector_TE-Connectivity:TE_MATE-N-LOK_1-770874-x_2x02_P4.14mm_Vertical (layer F.Cu) (at 73.66 134.239 270)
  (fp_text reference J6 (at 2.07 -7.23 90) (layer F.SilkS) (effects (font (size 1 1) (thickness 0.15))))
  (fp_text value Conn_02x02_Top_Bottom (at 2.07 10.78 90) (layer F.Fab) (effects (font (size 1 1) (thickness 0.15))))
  (fp_line (start -1.103302 -2.955) (end -2.955 -2.955) (layer F.SilkS) (width 0.12))
  (fp_line (start -2.955 -2.955) (end -2.955 7.095) (layer F.SilkS) (width 0.12))
  (fp_line (start -2.955 7.095) (end 0 7.095) (layer F.SilkS) (width 0.12))
  (fp_line (start 1.103302 -2.955) (end 7.095 -2.955) (layer F.SilkS) (width 0.12))
  (fp_line (start 7.095 -2.955) (end 7.095 7.095) (layer F.SilkS) (width 0.12))
  (fp_line (start 7.095 7.095) (end 0 7.095) (layer F.SilkS) (width 0.12))
  (fp_line (start -2.955 0.46) (end -4.255 0.46) (layer F.SilkS) (width 0.12))
  (fp_line (start -4.255 0.46) (end -4.255 3.68) (layer F.SilkS) (width 0.12))
  (fp_line (start -4.255 3.68) (end -2.955 3.68) (layer F.SilkS) (width 0.12))
  (fp_line (start 7.095 -2.955) (end 7.855 -2.955) (layer F.SilkS) (width 0.12))
  (fp_line (start 7.855 -2.955) (end 7.855 -1.595) (layer F.SilkS) (width 0.12))
  (fp_line (start 7.855 -1.595) (end 7.095 -1.595) (layer F.SilkS) (width 0.12))
  (fp_line (start 2.76 7.095) (end 2.76 9.686) (layer F.SilkS) (width 0.12))
  (fp_line (start 2.76 9.686) (end 5.52 9.686) (layer F.SilkS) (width 0.12))
  (fp_line (start 5.52 9.686) (end 5.52 7.095) (layer F.SilkS) (width 0.12))
  (fp_line (start 7.095 1.39) (end 7.855 1.39) (layer F.SilkS) (width 0.12))
  (fp_line (start 7.855 1.39) (end 7.855 2.75) (layer F.SilkS) (width 0.12))
  (fp_line (start 7.855 2.75) (end 7.095 2.75) (layer F.SilkS) (width 0.12))
  (fp_line (start 7.095 5.53) (end 7.855 5.53) (layer F.SilkS) (width 0.12))
  (fp_line (start 7.855 5.53) (end 7.855 6.89) (layer F.SilkS) (width 0.12))
  (fp_line (start 7.855 6.89) (end 7.095 6.89) (layer F.SilkS) (width 0.12))
  (fp_line (start -1.42066 -3.255) (end -3.255 -3.255) (layer F.SilkS) (width 0.12))
  (fp_line (start -3.255 -3.255) (end -3.255 -0.345) (layer F.SilkS) (width 0.12))
  (pad 1 thru_hole roundrect (at 0 0 270) (size 2.64 2.64) (drill 1.4) (layers *.Cu *.Mask) (roundrect_rratio 0.094697) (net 2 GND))
  (pad 2 thru_hole circle (at 0 4.14 270) (size 2.64 2.64) (drill 1.4) (layers *.Cu *.Mask) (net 2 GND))
  (pad 3 thru_hole circle (at 4.14 0 270) (size 2.64 2.64) (drill 1.4) (layers *.Cu *.Mask) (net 6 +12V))
  (pad 4 thru_hole circle (at 4.14 4.14 270) (size 2.64 2.64) (drill 1.4) (layers *.Cu *.Mask) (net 6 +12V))
  (pad "" np_thru_hole circle (at 0 -4.44 270) (size 3.18 3.18) (drill 3.18) (layers *.Cu *.Mask)))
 (gr_line (start 63.5 156.591) (end 63.5 70.993) (layer Edge.Cuts) (width 0.12))
 (gr_line (start 97.028 156.591) (end 63.5 156.591) (layer Edge.Cuts) (width 0.12))
 (gr_line (start 97.155 70.993) (end 97.028 156.591) (layer Edge.Cuts) (width 0.12))
 (gr_line (start 93.599 70.993) (end 97.155 70.993) (layer Edge.Cuts) (width 0.12))
 (gr_line (start 63.5 70.993) (end 93.599 70.993) (layer Edge.Cuts) (width 0.12))
 (segment (start 70.041762 102.388001) (end 72.315001 102.388001) (width 0.25) (layer F.Cu) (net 2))
 (segment (start 68.175001 102.388001) (end 70.041762 102.388001) (width 0.25) (layer F.Cu) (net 2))
 (segment (start 72.315001 100.52124) (end 72.315001 98.248001) (width 0.25) (layer F.Cu) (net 2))
 (segment (start 72.315001 102.388001) (end 72.315001 100.52124) (width 0.25) (layer F.Cu) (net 2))
 (segment (start 72.315001 96.38124) (end 72.315001 94.108001) (width 0.25) (layer F.Cu) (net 2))
 (segment (start 72.315001 98.248001) (end 72.315001 96.38124) (width 0.25) (layer F.Cu) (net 2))
 (segment (start 70.44824 94.108001) (end 68.175001 94.108001) (width 0.25) (layer F.Cu) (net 2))
 (segment (start 72.315001 94.108001) (end 70.44824 94.108001) (width 0.25) (layer F.Cu) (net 2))
 (segment (start 72.315001 92.24124) (end 72.315001 89.968001) (width 0.25) (layer F.Cu) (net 2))
 (segment (start 72.315001 94.108001) (end 72.315001 92.24124) (width 0.25) (layer F.Cu) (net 2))
 (segment (start 72.315001 88.10124) (end 72.315001 85.828001) (width 0.25) (layer F.Cu) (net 2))
 (segment (start 72.315001 89.968001) (end 72.315001 88.10124) (width 0.25) (layer F.Cu) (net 2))
 (segment (start 70.44824 85.828001) (end 68.175001 85.828001) (width 0.25) (layer F.Cu) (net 2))
 (segment (start 72.315001 85.828001) (end 70.44824 85.828001) (width 0.25) (layer F.Cu) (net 2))
 (segment (start 90.473999 98.248001) (end 91.313 97.409) (width 0.25) (layer F.Cu) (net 2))
 (segment (start 72.315001 98.248001) (end 90.473999 98.248001) (width 0.25) (layer F.Cu) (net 2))
 (segment (start 69.52 147.193) (end 73.66 147.193) (width 2) (layer F.Cu) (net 2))
 (segment (start 69.52 134.239) (end 73.66 134.239) (width 2) (layer F.Cu) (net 2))
 (segment (start 77.724 143.129) (end 89.535 143.129) (width 2) (layer F.Cu) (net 2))
 (segment (start 73.66 147.193) (end 77.724 143.129) (width 2) (layer F.Cu) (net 2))
 (segment (start 84.455 123.444) (end 73.66 134.239) (width 2) (layer F.Cu) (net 2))
 (segment (start 89.535 123.444) (end 84.455 123.444) (width 2) (layer F.Cu) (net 2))
 (segment (start 73.635 103.708) (end 72.315001 102.388001) (width 0.25) (layer F.Cu) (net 2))
 (segment (start 73.960002 104.033002) (end 73.635 103.708) (width 0.25) (layer F.Cu) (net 2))
 (segment (start 73.960002 121.443) (end 73.960002 104.033002) (width 0.25) (layer F.Cu) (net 2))
 (segment (start 72.315001 123.088001) (end 73.960002 121.443) (width 0.25) (layer F.Cu) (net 2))
 (segment (start 72.315001 118.948001) (end 72.315001 114.808001) (width 0.25) (layer F.Cu) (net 3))
 (segment (start 72.315001 112.94124) (end 72.315001 110.668001) (width 0.25) (layer F.Cu) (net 3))
 (segment (start 72.315001 114.808001) (end 72.315001 112.94124) (width 0.25) (layer F.Cu) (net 3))
 (segment (start 70.67 109.023) (end 70.995002 109.348002) (width 0.25) (layer F.Cu) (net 3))
 (segment (start 70.995002 109.348002) (end 72.315001 110.668001) (width 0.25) (layer F.Cu) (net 3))
 (segment (start 70.67 105.7384) (end 70.67 109.023) (width 0.25) (layer F.Cu) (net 3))
 (segment (start 69.8146 104.883) (end 70.67 105.7384) (width 0.25) (layer F.Cu) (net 3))
 (segment (start 67.3854 104.883) (end 69.8146 104.883) (width 0.25) (layer F.Cu) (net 3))
 (segment (start 66.53 104.0276) (end 67.3854 104.883) (width 0.25) (layer F.Cu) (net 3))
 (segment (start 66.53 99.893002) (end 66.53 104.0276) (width 0.25) (layer F.Cu) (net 3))
 (segment (start 68.175001 98.248001) (end 66.53 99.893002) (width 0.25) (layer F.Cu) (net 3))
 (segment (start 66.855002 96.928002) (end 68.175001 98.248001) (width 0.25) (layer F.Cu) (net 3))
 (segment (start 66.53 96.603) (end 66.855002 96.928002) (width 0.25) (layer F.Cu) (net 3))
 (segment (start 66.53 91.613002) (end 66.53 96.603) (width 0.25) (layer F.Cu) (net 3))
 (segment (start 68.175001 89.968001) (end 66.53 91.613002) (width 0.25) (layer F.Cu) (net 3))
 (segment (start 89.793 89.789) (end 91.313 89.789) (width 0.25) (layer F.Cu) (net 3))
 (segment (start 84.187 84.183) (end 89.793 89.789) (width 0.25) (layer F.Cu) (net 3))
 (segment (start 67.3854 84.183) (end 84.187 84.183) (width 0.25) (layer F.Cu) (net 3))
 (segment (start 66.53 85.0384) (end 67.3854 84.183) (width 0.25) (layer F.Cu) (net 3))
 (segment (start 66.53 88.323) (end 66.53 85.0384) (width 0.25) (layer F.Cu) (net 3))
 (segment (start 68.175001 89.968001) (end 66.53 88.323) (width 0.25) (layer F.Cu) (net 3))
 (segment (start 69.52 151.333) (end 73.66 151.333) (width 2) (layer F.Cu) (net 6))
 (segment (start 69.52 138.379) (end 73.66 138.379) (width 2) (layer F.Cu) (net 6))
 (segment (start 88.951 151.333) (end 89.535 150.749) (width 2) (layer F.Cu) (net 6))
 (segment (start 73.66 151.333) (end 88.951 151.333) (width 2) (layer F.Cu) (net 6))
 (segment (start 89.535 134.334) (end 89.535 131.064) (width 2) (layer F.Cu) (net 6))
 (segment (start 85.49 138.379) (end 89.535 134.334) (width 2) (layer F.Cu) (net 6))
 (segment (start 73.66 138.379) (end 85.49 138.379) (width 2) (layer F.Cu) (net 6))
 (segment (start 68.175001 117.08124) (end 68.175001 114.808001) (width 0.25) (layer F.Cu) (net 6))
 (segment (start 68.175001 118.948001) (end 68.175001 117.08124) (width 0.25) (layer F.Cu) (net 6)))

